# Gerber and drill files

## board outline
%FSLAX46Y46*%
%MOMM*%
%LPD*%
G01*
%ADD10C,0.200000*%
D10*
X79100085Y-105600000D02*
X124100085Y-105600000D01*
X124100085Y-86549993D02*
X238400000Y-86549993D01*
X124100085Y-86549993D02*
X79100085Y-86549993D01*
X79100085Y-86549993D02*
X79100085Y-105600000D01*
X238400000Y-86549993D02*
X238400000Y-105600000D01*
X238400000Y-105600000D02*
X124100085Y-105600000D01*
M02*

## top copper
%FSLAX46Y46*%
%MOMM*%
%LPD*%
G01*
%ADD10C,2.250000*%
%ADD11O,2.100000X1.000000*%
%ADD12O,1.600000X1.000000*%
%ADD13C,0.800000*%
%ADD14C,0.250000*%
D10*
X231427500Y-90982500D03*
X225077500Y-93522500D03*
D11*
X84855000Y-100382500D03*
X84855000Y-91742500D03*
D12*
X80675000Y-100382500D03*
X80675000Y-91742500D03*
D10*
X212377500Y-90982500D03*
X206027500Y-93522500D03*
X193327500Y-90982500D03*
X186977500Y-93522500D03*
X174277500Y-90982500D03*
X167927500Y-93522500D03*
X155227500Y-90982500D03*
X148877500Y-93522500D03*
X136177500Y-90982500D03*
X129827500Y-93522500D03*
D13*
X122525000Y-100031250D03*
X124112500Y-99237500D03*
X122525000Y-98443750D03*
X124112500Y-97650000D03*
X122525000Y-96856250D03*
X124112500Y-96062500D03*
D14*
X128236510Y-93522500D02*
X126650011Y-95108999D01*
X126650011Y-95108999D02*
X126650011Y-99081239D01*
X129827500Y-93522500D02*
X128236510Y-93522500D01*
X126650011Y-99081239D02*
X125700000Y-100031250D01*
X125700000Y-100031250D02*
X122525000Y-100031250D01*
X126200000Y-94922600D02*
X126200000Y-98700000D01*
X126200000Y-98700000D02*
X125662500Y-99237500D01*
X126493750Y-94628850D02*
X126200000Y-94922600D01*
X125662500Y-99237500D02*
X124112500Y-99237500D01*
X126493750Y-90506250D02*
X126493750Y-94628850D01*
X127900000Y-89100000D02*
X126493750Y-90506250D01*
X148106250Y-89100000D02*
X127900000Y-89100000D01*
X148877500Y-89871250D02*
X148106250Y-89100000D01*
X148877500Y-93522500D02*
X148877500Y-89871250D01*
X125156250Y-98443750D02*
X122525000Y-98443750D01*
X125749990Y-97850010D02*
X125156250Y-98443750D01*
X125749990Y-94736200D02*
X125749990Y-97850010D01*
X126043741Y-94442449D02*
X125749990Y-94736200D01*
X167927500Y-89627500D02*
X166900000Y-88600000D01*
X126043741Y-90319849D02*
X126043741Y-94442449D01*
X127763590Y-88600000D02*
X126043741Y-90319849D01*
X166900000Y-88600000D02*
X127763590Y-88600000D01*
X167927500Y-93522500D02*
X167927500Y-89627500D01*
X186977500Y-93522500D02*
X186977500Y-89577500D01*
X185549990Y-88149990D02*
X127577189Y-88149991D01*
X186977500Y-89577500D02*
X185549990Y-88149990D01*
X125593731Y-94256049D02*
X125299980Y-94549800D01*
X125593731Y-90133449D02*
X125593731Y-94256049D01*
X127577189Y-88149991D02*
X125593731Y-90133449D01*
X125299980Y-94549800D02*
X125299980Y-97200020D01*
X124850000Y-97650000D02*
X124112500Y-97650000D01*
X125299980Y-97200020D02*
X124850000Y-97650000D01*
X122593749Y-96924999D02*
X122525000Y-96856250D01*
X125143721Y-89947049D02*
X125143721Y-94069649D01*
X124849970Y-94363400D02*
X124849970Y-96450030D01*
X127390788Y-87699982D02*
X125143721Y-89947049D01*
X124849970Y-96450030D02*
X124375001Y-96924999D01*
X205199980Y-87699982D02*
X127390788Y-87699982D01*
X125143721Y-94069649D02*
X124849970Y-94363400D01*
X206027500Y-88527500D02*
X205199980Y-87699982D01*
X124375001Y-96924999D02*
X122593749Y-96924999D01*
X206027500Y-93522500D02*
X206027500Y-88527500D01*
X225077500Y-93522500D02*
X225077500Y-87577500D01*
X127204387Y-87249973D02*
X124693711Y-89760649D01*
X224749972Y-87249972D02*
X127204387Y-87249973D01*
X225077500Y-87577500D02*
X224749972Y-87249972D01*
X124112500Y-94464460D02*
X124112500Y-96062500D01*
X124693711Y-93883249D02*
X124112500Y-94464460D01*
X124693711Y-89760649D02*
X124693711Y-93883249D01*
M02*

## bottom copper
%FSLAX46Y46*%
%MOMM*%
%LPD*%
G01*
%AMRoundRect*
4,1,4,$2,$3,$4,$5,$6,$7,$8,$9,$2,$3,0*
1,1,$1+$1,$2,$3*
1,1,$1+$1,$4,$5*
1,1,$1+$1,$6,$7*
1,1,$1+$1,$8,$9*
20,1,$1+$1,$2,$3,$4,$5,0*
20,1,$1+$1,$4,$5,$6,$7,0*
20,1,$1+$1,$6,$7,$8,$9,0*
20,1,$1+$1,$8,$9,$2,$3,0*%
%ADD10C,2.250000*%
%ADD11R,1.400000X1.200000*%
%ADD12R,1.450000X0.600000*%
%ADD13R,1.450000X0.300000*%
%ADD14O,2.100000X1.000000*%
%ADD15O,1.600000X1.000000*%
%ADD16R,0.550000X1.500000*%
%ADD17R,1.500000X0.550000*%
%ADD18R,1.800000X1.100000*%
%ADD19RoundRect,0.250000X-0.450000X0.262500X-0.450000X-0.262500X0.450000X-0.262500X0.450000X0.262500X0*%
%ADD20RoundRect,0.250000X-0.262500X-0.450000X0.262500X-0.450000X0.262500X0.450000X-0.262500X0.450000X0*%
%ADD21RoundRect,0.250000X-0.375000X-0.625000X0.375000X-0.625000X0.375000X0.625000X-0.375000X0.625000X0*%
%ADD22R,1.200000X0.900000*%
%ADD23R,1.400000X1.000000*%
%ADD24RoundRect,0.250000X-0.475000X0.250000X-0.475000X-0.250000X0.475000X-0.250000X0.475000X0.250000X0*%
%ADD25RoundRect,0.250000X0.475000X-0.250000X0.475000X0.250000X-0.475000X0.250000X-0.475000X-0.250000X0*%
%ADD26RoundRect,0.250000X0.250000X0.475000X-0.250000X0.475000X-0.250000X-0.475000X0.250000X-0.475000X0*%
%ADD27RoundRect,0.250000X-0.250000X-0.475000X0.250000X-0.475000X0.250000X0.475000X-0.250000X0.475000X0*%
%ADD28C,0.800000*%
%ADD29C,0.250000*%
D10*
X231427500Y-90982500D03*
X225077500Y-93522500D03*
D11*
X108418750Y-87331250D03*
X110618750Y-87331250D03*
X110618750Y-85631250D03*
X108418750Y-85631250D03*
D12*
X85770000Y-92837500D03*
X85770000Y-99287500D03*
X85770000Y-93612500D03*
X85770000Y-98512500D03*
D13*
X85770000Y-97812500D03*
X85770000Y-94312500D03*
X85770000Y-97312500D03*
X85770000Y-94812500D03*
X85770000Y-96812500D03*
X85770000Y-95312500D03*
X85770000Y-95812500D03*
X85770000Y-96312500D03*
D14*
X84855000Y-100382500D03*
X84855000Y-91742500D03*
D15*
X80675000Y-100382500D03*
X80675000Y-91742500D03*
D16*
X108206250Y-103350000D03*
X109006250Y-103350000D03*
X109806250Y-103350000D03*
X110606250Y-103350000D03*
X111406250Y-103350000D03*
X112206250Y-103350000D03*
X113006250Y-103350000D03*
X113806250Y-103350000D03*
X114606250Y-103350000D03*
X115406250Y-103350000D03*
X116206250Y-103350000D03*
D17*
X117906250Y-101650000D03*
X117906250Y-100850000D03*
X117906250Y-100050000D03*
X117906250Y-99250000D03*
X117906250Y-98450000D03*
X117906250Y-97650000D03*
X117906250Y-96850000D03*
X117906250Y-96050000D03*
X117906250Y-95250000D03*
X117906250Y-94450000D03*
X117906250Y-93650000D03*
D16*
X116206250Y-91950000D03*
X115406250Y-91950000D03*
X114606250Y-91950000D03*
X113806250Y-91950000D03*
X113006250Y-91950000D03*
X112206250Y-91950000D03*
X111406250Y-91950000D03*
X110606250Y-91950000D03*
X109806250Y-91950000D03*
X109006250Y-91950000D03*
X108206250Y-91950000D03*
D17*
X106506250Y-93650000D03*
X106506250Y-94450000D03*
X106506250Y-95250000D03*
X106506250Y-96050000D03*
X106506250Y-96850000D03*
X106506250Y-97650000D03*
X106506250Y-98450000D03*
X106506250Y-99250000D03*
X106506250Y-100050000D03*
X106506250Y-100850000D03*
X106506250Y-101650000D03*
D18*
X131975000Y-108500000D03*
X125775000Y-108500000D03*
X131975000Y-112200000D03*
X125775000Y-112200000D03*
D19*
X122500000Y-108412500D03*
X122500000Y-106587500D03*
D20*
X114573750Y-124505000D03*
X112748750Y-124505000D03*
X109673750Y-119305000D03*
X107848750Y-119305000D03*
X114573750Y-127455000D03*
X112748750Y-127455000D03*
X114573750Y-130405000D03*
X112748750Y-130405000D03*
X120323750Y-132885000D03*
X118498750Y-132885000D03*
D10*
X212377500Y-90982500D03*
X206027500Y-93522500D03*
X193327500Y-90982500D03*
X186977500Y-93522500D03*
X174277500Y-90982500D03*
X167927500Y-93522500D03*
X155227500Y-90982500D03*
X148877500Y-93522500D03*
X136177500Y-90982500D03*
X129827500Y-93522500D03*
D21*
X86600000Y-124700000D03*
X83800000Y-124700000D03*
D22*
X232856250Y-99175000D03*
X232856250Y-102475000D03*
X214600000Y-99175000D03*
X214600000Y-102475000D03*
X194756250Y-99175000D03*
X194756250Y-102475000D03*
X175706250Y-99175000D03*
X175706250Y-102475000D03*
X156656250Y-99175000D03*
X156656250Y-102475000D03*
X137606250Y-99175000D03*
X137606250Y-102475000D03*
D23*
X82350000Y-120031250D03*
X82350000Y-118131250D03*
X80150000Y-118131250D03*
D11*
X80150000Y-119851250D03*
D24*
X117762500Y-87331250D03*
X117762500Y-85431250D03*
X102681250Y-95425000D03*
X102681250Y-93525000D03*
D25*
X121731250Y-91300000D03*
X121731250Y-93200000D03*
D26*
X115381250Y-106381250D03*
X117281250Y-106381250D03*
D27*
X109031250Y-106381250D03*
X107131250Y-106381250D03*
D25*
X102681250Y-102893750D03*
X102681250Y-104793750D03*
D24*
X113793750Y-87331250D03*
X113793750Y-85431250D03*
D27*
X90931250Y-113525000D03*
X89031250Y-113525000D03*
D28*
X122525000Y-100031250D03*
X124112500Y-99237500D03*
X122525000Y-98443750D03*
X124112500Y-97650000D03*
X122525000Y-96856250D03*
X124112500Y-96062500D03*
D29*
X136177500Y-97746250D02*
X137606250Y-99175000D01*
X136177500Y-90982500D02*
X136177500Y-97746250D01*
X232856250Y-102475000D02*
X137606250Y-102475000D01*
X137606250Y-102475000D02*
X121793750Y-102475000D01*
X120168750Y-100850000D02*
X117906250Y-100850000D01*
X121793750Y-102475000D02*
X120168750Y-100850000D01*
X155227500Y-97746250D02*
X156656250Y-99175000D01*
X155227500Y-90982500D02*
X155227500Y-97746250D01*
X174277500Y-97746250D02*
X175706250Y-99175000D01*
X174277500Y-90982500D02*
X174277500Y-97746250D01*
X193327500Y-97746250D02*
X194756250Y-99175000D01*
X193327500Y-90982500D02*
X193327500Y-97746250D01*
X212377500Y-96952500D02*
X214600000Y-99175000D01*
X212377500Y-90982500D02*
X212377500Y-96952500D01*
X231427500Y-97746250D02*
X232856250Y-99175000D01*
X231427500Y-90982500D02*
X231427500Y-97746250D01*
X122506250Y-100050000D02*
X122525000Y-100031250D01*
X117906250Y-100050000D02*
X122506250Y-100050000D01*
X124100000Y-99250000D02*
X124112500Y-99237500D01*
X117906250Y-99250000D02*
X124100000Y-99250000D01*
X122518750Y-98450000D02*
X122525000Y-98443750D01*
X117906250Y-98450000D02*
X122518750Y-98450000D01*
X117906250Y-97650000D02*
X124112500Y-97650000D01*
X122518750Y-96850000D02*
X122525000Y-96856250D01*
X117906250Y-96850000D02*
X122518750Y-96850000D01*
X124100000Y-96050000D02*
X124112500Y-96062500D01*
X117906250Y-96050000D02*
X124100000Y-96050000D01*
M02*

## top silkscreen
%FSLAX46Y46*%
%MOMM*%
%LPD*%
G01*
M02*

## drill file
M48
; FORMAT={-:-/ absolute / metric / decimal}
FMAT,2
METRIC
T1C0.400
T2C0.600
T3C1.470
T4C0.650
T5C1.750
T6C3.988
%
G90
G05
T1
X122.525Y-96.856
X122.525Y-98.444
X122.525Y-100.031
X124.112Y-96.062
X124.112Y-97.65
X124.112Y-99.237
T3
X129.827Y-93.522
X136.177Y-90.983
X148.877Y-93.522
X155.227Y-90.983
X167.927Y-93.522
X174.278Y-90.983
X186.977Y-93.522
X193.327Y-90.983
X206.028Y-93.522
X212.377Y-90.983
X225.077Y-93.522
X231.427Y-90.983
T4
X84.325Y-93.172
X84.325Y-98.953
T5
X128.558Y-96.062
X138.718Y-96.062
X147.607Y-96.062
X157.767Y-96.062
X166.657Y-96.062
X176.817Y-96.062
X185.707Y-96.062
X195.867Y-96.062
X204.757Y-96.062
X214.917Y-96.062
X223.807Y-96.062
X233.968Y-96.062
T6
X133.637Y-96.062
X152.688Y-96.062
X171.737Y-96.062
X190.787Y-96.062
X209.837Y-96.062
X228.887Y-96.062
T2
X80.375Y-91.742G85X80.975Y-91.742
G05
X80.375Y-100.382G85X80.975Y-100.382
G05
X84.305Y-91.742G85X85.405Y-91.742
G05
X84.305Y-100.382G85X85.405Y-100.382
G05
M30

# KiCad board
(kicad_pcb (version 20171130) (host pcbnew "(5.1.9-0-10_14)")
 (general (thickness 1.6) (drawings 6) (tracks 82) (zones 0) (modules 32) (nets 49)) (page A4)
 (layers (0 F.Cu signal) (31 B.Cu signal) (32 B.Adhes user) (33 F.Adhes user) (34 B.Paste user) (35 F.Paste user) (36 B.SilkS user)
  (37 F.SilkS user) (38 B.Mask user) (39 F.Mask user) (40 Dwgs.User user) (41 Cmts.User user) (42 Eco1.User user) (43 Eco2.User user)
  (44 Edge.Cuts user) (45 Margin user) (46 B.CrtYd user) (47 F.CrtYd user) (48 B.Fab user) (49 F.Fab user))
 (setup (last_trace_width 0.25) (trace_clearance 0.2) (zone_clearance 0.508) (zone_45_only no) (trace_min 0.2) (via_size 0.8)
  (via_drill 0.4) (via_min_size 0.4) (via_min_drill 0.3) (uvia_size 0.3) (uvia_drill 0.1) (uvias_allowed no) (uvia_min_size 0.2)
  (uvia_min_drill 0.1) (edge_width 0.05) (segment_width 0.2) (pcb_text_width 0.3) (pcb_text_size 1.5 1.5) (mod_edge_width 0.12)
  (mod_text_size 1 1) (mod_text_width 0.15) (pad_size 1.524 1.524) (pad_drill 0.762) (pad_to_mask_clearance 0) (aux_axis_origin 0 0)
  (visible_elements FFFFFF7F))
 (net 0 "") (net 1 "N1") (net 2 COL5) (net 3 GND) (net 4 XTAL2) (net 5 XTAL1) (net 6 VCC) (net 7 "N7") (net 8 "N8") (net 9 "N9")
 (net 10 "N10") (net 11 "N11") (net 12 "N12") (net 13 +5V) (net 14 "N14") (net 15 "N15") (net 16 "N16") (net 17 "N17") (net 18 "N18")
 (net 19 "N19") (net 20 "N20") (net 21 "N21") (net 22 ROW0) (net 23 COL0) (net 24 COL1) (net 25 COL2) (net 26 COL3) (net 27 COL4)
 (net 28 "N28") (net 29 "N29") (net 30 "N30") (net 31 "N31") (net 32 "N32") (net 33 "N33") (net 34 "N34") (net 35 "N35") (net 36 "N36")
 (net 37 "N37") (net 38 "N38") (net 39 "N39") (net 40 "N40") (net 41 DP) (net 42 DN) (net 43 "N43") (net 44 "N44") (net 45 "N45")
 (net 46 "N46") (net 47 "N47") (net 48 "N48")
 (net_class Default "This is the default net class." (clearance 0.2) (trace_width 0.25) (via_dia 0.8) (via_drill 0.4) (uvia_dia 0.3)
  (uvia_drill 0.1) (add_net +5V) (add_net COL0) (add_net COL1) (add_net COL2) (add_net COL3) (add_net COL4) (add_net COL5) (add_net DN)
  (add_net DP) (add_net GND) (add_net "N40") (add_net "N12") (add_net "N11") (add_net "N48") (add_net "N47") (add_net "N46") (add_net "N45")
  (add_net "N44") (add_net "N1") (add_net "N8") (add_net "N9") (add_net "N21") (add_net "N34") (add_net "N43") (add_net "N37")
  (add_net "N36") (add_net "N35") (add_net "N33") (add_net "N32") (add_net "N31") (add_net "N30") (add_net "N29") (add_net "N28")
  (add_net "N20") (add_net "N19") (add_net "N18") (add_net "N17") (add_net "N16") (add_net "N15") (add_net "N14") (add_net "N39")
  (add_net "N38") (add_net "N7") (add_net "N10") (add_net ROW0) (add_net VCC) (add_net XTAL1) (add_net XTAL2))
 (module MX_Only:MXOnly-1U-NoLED (layer F.Cu) (at 228.8875 96.0625)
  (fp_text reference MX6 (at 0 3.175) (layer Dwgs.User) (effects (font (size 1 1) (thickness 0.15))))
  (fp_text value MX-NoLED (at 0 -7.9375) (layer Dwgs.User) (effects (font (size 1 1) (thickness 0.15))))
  (pad 2 thru_hole circle (at 2.54 -5.08) (size 2.25 2.25) (drill 1.47) (layers *.Cu B.Mask) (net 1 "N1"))
  (pad "" np_thru_hole circle (at 0 0) (size 3.9878 3.9878) (drill 3.9878) (layers *.Cu *.Mask))
  (pad 1 thru_hole circle (at -3.81 -2.54) (size 2.25 2.25) (drill 1.47) (layers *.Cu B.Mask) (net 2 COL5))
  (pad "" np_thru_hole circle (at -5.08 0 48.0996) (size 1.75 1.75) (drill 1.75) (layers *.Cu *.Mask))
  (pad "" np_thru_hole circle (at 5.08 0 48.0996) (size 1.75 1.75) (drill 1.75) (layers *.Cu *.Mask)))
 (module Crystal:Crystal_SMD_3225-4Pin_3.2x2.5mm (layer B.Cu) (at 109.51875 86.48125)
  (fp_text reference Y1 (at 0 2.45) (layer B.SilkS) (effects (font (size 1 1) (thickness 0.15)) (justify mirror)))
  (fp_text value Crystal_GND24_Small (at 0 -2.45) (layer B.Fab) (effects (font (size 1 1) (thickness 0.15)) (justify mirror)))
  (pad 4 smd rect (at -1.1 0.85) (size 1.4 1.2) (layers B.Cu B.Paste B.Mask) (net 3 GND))
  (pad 3 smd rect (at 1.1 0.85) (size 1.4 1.2) (layers B.Cu B.Paste B.Mask) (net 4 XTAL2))
  (pad 2 smd rect (at 1.1 -0.85) (size 1.4 1.2) (layers B.Cu B.Paste B.Mask) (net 3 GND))
  (pad 1 smd rect (at -1.1 -0.85) (size 1.4 1.2) (layers B.Cu B.Paste B.Mask) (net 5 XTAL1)))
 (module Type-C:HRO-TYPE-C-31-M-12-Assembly (layer B.Cu) (at 78.075 96.0625 90)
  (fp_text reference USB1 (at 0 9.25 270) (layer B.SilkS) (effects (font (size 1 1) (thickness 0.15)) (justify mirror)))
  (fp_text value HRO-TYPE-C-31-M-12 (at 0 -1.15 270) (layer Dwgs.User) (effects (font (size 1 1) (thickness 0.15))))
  (pad 12 smd rect (at 3.225 7.695 90) (size 0.6 1.45) (layers B.Cu B.Paste B.Mask) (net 3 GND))
  (pad 1 smd rect (at -3.225 7.695 90) (size 0.6 1.45) (layers B.Cu B.Paste B.Mask) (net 3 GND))
  (pad 11 smd rect (at 2.45 7.695 90) (size 0.6 1.45) (layers B.Cu B.Paste B.Mask) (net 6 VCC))
  (pad 2 smd rect (at -2.45 7.695 90) (size 0.6 1.45) (layers B.Cu B.Paste B.Mask) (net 6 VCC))
  (pad 3 smd rect (at -1.75 7.695 90) (size 0.3 1.45) (layers B.Cu B.Paste B.Mask) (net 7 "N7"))
  (pad 10 smd rect (at 1.75 7.695 90) (size 0.3 1.45) (layers B.Cu B.Paste B.Mask) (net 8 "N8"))
  (pad 4 smd rect (at -1.25 7.695 90) (size 0.3 1.45) (layers B.Cu B.Paste B.Mask) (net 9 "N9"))
  (pad 9 smd rect (at 1.25 7.695 90) (size 0.3 1.45) (layers B.Cu B.Paste B.Mask) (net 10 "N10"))
  (pad 5 smd rect (at -0.75 7.695 90) (size 0.3 1.45) (layers B.Cu B.Paste B.Mask) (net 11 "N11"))
  (pad 8 smd rect (at 0.75 7.695 90) (size 0.3 1.45) (layers B.Cu B.Paste B.Mask) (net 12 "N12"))
  (pad 7 smd rect (at 0.25 7.695 90) (size 0.3 1.45) (layers B.Cu B.Paste B.Mask) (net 11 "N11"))
  (pad 6 smd rect (at -0.25 7.695 90) (size 0.3 1.45) (layers B.Cu B.Paste B.Mask) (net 12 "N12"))
  (pad "" np_thru_hole circle (at 2.89 6.25 90) (size 0.65 0.65) (drill 0.65) (layers *.Cu *.Mask))
  (pad "" np_thru_hole circle (at -2.89 6.25 90) (size 0.65 0.65) (drill 0.65) (layers *.Cu *.Mask))
  (pad 13 thru_hole oval (at -4.32 6.78 90) (size 1 2.1) (drill oval 0.6 1.7) (layers *.Cu *.Mask) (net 3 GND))
  (pad 13 thru_hole oval (at 4.32 6.78 90) (size 1 2.1) (drill oval 0.6 1.7) (layers *.Cu *.Mask) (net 3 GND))
  (pad 13 thru_hole oval (at -4.32 2.6 90) (size 1 1.6) (drill oval 0.6 1.2) (layers *.Cu *.Mask) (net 3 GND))
  (pad 13 thru_hole oval (at 4.32 2.6 90) (size 1 1.6) (drill oval 0.6 1.2) (layers *.Cu *.Mask) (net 3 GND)))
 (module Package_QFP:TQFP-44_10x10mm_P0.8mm (layer B.Cu) (at 112.20625 97.65)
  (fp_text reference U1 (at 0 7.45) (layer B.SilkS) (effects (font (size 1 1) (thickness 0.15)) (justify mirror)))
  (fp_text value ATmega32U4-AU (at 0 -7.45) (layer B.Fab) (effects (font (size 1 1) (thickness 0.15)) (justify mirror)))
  (pad 44 smd rect (at -4 5.7 270) (size 1.5 0.55) (layers B.Cu B.Paste B.Mask) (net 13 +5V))
  (pad 43 smd rect (at -3.2 5.7 270) (size 1.5 0.55) (layers B.Cu B.Paste B.Mask) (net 3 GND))
  (pad 42 smd rect (at -2.4 5.7 270) (size 1.5 0.55) (layers B.Cu B.Paste B.Mask) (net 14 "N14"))
  (pad 41 smd rect (at -1.6 5.7 270) (size 1.5 0.55) (layers B.Cu B.Paste B.Mask) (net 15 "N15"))
  (pad 40 smd rect (at -0.8 5.7 270) (size 1.5 0.55) (layers B.Cu B.Paste B.Mask) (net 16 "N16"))
  (pad 39 smd rect (at 0 5.7 270) (size 1.5 0.55) (layers B.Cu B.Paste B.Mask) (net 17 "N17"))
  (pad 38 smd rect (at 0.8 5.7 270) (size 1.5 0.55) (layers B.Cu B.Paste B.Mask) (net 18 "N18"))
  (pad 37 smd rect (at 1.6 5.7 270) (size 1.5 0.55) (layers B.Cu B.Paste B.Mask) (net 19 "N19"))
  (pad 36 smd rect (at 2.4 5.7 270) (size 1.5 0.55) (layers B.Cu B.Paste B.Mask) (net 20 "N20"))
  (pad 35 smd rect (at 3.2 5.7 270) (size 1.5 0.55) (layers B.Cu B.Paste B.Mask) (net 3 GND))
  (pad 34 smd rect (at 4 5.7 270) (size 1.5 0.55) (layers B.Cu B.Paste B.Mask) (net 13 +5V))
  (pad 33 smd rect (at 5.7 4) (size 1.5 0.55) (layers B.Cu B.Paste B.Mask) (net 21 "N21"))
  (pad 32 smd rect (at 5.7 3.2) (size 1.5 0.55) (layers B.Cu B.Paste B.Mask) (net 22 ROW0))
  (pad 31 smd rect (at 5.7 2.4) (size 1.5 0.55) (layers B.Cu B.Paste B.Mask) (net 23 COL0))
  (pad 30 smd rect (at 5.7 1.6) (size 1.5 0.55) (layers B.Cu B.Paste B.Mask) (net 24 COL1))
  (pad 29 smd rect (at 5.7 0.8) (size 1.5 0.55) (layers B.Cu B.Paste B.Mask) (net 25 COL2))
  (pad 28 smd rect (at 5.7 0) (size 1.5 0.55) (layers B.Cu B.Paste B.Mask) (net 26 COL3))
  (pad 27 smd rect (at 5.7 -0.8) (size 1.5 0.55) (layers B.Cu B.Paste B.Mask) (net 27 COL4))
  (pad 26 smd rect (at 5.7 -1.6) (size 1.5 0.55) (layers B.Cu B.Paste B.Mask) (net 2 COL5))
  (pad 25 smd rect (at 5.7 -2.4) (size 1.5 0.55) (layers B.Cu B.Paste B.Mask) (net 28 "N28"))
  (pad 24 smd rect (at 5.7 -3.2) (size 1.5 0.55) (layers B.Cu B.Paste B.Mask) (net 13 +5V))
  (pad 23 smd rect (at 5.7 -4) (size 1.5 0.55) (layers B.Cu B.Paste B.Mask) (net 3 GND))
  (pad 22 smd rect (at 4 -5.7 270) (size 1.5 0.55) (layers B.Cu B.Paste B.Mask) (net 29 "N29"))
  (pad 21 smd rect (at 3.2 -5.7 270) (size 1.5 0.55) (layers B.Cu B.Paste B.Mask) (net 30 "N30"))
  (pad 20 smd rect (at 2.4 -5.7 270) (size 1.5 0.55) (layers B.Cu B.Paste B.Mask) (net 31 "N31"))
  (pad 19 smd rect (at 1.6 -5.7 270) (size 1.5 0.55) (layers B.Cu B.Paste B.Mask) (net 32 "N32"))
  (pad 18 smd rect (at 0.8 -5.7 270) (size 1.5 0.55) (layers B.Cu B.Paste B.Mask) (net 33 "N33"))
  (pad 17 smd rect (at 0 -5.7 270) (size 1.5 0.55) (layers B.Cu B.Paste B.Mask) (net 5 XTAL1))
  (pad 16 smd rect (at -0.8 -5.7 270) (size 1.5 0.55) (layers B.Cu B.Paste B.Mask) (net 4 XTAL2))
  (pad 15 smd rect (at -1.6 -5.7 270) (size 1.5 0.55) (layers B.Cu B.Paste B.Mask) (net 3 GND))
  (pad 14 smd rect (at -2.4 -5.7 270) (size 1.5 0.55) (layers B.Cu B.Paste B.Mask) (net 13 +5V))
  (pad 13 smd rect (at -3.2 -5.7 270) (size 1.5 0.55) (layers B.Cu B.Paste B.Mask) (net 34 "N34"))
  (pad 12 smd rect (at -4 -5.7 270) (size 1.5 0.55) (layers B.Cu B.Paste B.Mask) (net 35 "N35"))
  (pad 11 smd rect (at -5.7 -4) (size 1.5 0.55) (layers B.Cu B.Paste B.Mask) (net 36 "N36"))
  (pad 10 smd rect (at -5.7 -3.2) (size 1.5 0.55) (layers B.Cu B.Paste B.Mask) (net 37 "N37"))
  (pad 9 smd rect (at -5.7 -2.4) (size 1.5 0.55) (layers B.Cu B.Paste B.Mask) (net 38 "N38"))
  (pad 8 smd rect (at -5.7 -1.6) (size 1.5 0.55) (layers B.Cu B.Paste B.Mask) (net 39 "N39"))
  (pad 7 smd rect (at -5.7 -0.8) (size 1.5 0.55) (layers B.Cu B.Paste B.Mask) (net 13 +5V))
  (pad 6 smd rect (at -5.7 0) (size 1.5 0.55) (layers B.Cu B.Paste B.Mask) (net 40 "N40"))
  (pad 5 smd rect (at -5.7 0.8) (size 1.5 0.55) (layers B.Cu B.Paste B.Mask) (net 3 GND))
  (pad 4 smd rect (at -5.7 1.6) (size 1.5 0.55) (layers B.Cu B.Paste B.Mask) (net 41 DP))
  (pad 3 smd rect (at -5.7 2.4) (size 1.5 0.55) (layers B.Cu B.Paste B.Mask) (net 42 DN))
  (pad 2 smd rect (at -5.7 3.2) (size 1.5 0.55) (layers B.Cu B.Paste B.Mask) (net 13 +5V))
  (pad 1 smd rect (at -5.7 4) (size 1.5 0.55) (layers B.Cu B.Paste B.Mask) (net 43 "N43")))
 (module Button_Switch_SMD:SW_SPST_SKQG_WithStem (layer B.Cu) (at 128.875 110.35)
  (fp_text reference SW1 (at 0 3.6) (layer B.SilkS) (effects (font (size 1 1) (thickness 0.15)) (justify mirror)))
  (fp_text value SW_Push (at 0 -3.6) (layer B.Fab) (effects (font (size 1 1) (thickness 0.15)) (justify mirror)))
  (pad 2 smd rect (at 3.1 -1.85) (size 1.8 1.1) (layers B.Cu B.Paste B.Mask) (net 34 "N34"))
  (pad 2 smd rect (at -3.1 -1.85) (size 1.8 1.1) (layers B.Cu B.Paste B.Mask) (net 34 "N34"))
  (pad 1 smd rect (at 3.1 1.85) (size 1.8 1.1) (layers B.Cu B.Paste B.Mask) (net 3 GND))
  (pad 1 smd rect (at -3.1 1.85) (size 1.8 1.1) (layers B.Cu B.Paste B.Mask) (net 3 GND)))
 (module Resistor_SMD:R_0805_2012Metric (layer B.Cu) (at 122.5 107.5 270)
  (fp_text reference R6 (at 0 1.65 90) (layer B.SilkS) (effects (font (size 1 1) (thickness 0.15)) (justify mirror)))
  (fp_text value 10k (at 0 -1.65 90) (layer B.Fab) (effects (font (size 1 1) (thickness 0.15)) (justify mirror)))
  (pad 2 smd roundrect (at 0.9125 0 270) (size 1.025 1.4) (layers B.Cu B.Paste B.Mask) (roundrect_rratio 0.243902) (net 34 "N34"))
  (pad 1 smd roundrect (at -0.9125 0 270) (size 1.025 1.4) (layers B.Cu B.Paste B.Mask) (roundrect_rratio 0.243902) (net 13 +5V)))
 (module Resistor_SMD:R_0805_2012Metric (layer B.Cu) (at 113.66125 124.505)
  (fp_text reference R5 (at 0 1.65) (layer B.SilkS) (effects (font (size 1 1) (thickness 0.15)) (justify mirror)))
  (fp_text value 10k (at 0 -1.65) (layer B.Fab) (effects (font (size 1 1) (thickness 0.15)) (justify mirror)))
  (pad 2 smd roundrect (at 0.9125 0) (size 1.025 1.4) (layers B.Cu B.Paste B.Mask) (roundrect_rratio 0.243902) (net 21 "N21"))
  (pad 1 smd roundrect (at -0.9125 0) (size 1.025 1.4) (layers B.Cu B.Paste B.Mask) (roundrect_rratio 0.243902) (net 3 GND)))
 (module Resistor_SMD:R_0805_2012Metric (layer B.Cu) (at 108.76125 119.305)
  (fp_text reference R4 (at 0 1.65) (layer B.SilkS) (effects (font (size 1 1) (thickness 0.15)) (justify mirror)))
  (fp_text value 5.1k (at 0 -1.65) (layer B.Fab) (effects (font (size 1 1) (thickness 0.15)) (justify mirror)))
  (pad 2 smd roundrect (at 0.9125 0) (size 1.025 1.4) (layers B.Cu B.Paste B.Mask) (roundrect_rratio 0.243902) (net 9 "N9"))
  (pad 1 smd roundrect (at -0.9125 0) (size 1.025 1.4) (layers B.Cu B.Paste B.Mask) (roundrect_rratio 0.243902) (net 3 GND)))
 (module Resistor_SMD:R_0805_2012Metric (layer B.Cu) (at 113.66125 127.455)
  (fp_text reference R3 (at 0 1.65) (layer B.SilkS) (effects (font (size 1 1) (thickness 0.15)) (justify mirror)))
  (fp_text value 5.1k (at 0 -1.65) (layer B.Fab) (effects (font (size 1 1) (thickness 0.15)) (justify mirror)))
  (pad 2 smd roundrect (at 0.9125 0) (size 1.025 1.4) (layers B.Cu B.Paste B.Mask) (roundrect_rratio 0.243902) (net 8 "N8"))
  (pad 1 smd roundrect (at -0.9125 0) (size 1.025 1.4) (layers B.Cu B.Paste B.Mask) (roundrect_rratio 0.243902) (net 3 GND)))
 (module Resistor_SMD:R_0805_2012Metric (layer B.Cu) (at 113.66125 130.405)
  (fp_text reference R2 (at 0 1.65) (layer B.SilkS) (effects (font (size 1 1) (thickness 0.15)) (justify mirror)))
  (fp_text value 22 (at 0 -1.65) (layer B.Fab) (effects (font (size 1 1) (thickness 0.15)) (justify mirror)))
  (pad 2 smd roundrect (at 0.9125 0) (size 1.025 1.4) (layers B.Cu B.Paste B.Mask) (roundrect_rratio 0.243902) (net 41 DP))
  (pad 1 smd roundrect (at -0.9125 0) (size 1.025 1.4) (layers B.Cu B.Paste B.Mask) (roundrect_rratio 0.243902) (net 12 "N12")))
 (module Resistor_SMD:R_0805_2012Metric (layer B.Cu) (at 119.41125 132.885)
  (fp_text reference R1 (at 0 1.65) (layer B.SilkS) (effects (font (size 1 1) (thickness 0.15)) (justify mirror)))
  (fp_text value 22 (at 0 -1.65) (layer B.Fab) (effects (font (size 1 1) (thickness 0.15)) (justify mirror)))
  (pad 2 smd roundrect (at 0.9125 0) (size 1.025 1.4) (layers B.Cu B.Paste B.Mask) (roundrect_rratio 0.243902) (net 42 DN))
  (pad 1 smd roundrect (at -0.9125 0) (size 1.025 1.4) (layers B.Cu B.Paste B.Mask) (roundrect_rratio 0.243902) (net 11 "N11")))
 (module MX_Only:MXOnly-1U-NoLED (layer F.Cu) (at 209.8375 96.0625)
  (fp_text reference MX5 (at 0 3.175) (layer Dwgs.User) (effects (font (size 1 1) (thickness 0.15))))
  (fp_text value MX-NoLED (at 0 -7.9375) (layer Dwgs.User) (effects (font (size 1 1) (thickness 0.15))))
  (pad 2 thru_hole circle (at 2.54 -5.08) (size 2.25 2.25) (drill 1.47) (layers *.Cu B.Mask) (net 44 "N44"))
  (pad "" np_thru_hole circle (at 0 0) (size 3.9878 3.9878) (drill 3.9878) (layers *.Cu *.Mask))
  (pad 1 thru_hole circle (at -3.81 -2.54) (size 2.25 2.25) (drill 1.47) (layers *.Cu B.Mask) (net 27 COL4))
  (pad "" np_thru_hole circle (at -5.08 0 48.0996) (size 1.75 1.75) (drill 1.75) (layers *.Cu *.Mask))
  (pad "" np_thru_hole circle (at 5.08 0 48.0996) (size 1.75 1.75) (drill 1.75) (layers *.Cu *.Mask)))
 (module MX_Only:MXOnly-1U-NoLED (layer F.Cu) (at 190.7875 96.0625)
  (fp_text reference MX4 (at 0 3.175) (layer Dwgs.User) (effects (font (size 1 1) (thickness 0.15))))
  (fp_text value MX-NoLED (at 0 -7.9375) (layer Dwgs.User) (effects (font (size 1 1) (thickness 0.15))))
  (pad 2 thru_hole circle (at 2.54 -5.08) (size 2.25 2.25) (drill 1.47) (layers *.Cu B.Mask) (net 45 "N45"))
  (pad "" np_thru_hole circle (at 0 0) (size 3.9878 3.9878) (drill 3.9878) (layers *.Cu *.Mask))
  (pad 1 thru_hole circle (at -3.81 -2.54) (size 2.25 2.25) (drill 1.47) (layers *.Cu B.Mask) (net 26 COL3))
  (pad "" np_thru_hole circle (at -5.08 0 48.0996) (size 1.75 1.75) (drill 1.75) (layers *.Cu *.Mask))
  (pad "" np_thru_hole circle (at 5.08 0 48.0996) (size 1.75 1.75) (drill 1.75) (layers *.Cu *.Mask)))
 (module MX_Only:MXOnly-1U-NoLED (layer F.Cu) (at 171.7375 96.0625)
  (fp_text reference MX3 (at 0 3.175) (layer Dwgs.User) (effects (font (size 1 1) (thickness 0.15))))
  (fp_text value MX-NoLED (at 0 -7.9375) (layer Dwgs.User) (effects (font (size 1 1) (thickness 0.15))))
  (pad 2 thru_hole circle (at 2.54 -5.08) (size 2.25 2.25) (drill 1.47) (layers *.Cu B.Mask) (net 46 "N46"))
  (pad "" np_thru_hole circle (at 0 0) (size 3.9878 3.9878) (drill 3.9878) (layers *.Cu *.Mask))
  (pad 1 thru_hole circle (at -3.81 -2.54) (size 2.25 2.25) (drill 1.47) (layers *.Cu B.Mask) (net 25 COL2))
  (pad "" np_thru_hole circle (at -5.08 0 48.0996) (size 1.75 1.75) (drill 1.75) (layers *.Cu *.Mask))
  (pad "" np_thru_hole circle (at 5.08 0 48.0996) (size 1.75 1.75) (drill 1.75) (layers *.Cu *.Mask)))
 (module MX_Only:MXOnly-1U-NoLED (layer F.Cu) (at 152.6875 96.0625)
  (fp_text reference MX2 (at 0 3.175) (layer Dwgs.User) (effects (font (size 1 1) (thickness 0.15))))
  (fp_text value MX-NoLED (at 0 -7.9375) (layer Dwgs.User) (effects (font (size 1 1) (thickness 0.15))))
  (pad 2 thru_hole circle (at 2.54 -5.08) (size 2.25 2.25) (drill 1.47) (layers *.Cu B.Mask) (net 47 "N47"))
  (pad "" np_thru_hole circle (at 0 0) (size 3.9878 3.9878) (drill 3.9878) (layers *.Cu *.Mask))
  (pad 1 thru_hole circle (at -3.81 -2.54) (size 2.25 2.25) (drill 1.47) (layers *.Cu B.Mask) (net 24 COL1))
  (pad "" np_thru_hole circle (at -5.08 0 48.0996) (size 1.75 1.75) (drill 1.75) (layers *.Cu *.Mask))
  (pad "" np_thru_hole circle (at 5.08 0 48.0996) (size 1.75 1.75) (drill 1.75) (layers *.Cu *.Mask)))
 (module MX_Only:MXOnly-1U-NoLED (layer F.Cu) (at 133.6375 96.0625)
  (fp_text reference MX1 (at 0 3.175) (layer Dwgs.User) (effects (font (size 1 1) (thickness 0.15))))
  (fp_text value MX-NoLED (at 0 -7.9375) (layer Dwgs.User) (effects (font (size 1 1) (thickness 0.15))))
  (pad 2 thru_hole circle (at 2.54 -5.08) (size 2.25 2.25) (drill 1.47) (layers *.Cu B.Mask) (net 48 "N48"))
  (pad "" np_thru_hole circle (at 0 0) (size 3.9878 3.9878) (drill 3.9878) (layers *.Cu *.Mask))
  (pad 1 thru_hole circle (at -3.81 -2.54) (size 2.25 2.25) (drill 1.47) (layers *.Cu B.Mask) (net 23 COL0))
  (pad "" np_thru_hole circle (at -5.08 0 48.0996) (size 1.75 1.75) (drill 1.75) (layers *.Cu *.Mask))
  (pad "" np_thru_hole circle (at 5.08 0 48.0996) (size 1.75 1.75) (drill 1.75) (layers *.Cu *.Mask)))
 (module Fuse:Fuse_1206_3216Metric (layer B.Cu) (at 85.2 124.7)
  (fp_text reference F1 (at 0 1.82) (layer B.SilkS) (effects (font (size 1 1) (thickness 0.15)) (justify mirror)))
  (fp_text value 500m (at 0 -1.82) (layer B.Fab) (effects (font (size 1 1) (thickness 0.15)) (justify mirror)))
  (pad 2 smd roundrect (at 1.4 0) (size 1.25 1.75) (layers B.Cu B.Paste B.Mask) (roundrect_rratio 0.2) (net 6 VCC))
  (pad 1 smd roundrect (at -1.4 0) (size 1.25 1.75) (layers B.Cu B.Paste B.Mask) (roundrect_rratio 0.2) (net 13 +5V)))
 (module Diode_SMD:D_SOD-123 (layer B.Cu) (at 232.85625 100.825 90)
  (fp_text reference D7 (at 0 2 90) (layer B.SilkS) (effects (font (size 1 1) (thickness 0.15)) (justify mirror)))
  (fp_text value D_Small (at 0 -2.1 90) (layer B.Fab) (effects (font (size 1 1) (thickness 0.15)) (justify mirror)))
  (pad 2 smd rect (at 1.65 0 90) (size 0.9 1.2) (layers B.Cu B.Paste B.Mask) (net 1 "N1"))
  (pad 1 smd rect (at -1.65 0 90) (size 0.9 1.2) (layers B.Cu B.Paste B.Mask) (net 22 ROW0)))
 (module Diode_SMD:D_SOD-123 (layer B.Cu) (at 214.6 100.825 90)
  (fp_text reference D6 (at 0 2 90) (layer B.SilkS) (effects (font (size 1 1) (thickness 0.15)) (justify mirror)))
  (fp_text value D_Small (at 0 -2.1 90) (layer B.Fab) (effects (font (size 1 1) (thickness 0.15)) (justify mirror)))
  (pad 2 smd rect (at 1.65 0 90) (size 0.9 1.2) (layers B.Cu B.Paste B.Mask) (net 44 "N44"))
  (pad 1 smd rect (at -1.65 0 90) (size 0.9 1.2) (layers B.Cu B.Paste B.Mask) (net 22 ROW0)))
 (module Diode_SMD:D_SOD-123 (layer B.Cu) (at 194.75625 100.825 90)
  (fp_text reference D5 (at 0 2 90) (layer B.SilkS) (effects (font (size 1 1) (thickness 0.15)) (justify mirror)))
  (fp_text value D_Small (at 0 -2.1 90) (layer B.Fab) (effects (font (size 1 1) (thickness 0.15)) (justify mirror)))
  (pad 2 smd rect (at 1.65 0 90) (size 0.9 1.2) (layers B.Cu B.Paste B.Mask) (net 45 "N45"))
  (pad 1 smd rect (at -1.65 0 90) (size 0.9 1.2) (layers B.Cu B.Paste B.Mask) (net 22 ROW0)))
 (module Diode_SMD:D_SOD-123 (layer B.Cu) (at 175.70625 100.825 90)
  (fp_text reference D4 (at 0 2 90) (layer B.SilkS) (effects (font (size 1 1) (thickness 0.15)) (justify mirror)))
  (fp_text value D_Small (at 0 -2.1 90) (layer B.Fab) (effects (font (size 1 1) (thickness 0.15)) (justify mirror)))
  (pad 2 smd rect (at 1.65 0 90) (size 0.9 1.2) (layers B.Cu B.Paste B.Mask) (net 46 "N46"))
  (pad 1 smd rect (at -1.65 0 90) (size 0.9 1.2) (layers B.Cu B.Paste B.Mask) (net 22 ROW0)))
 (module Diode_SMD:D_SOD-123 (layer B.Cu) (at 156.65625 100.825 90)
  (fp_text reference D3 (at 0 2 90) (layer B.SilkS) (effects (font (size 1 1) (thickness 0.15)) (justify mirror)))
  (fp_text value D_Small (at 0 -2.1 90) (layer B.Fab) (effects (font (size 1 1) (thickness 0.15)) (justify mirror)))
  (pad 2 smd rect (at 1.65 0 90) (size 0.9 1.2) (layers B.Cu B.Paste B.Mask) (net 47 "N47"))
  (pad 1 smd rect (at -1.65 0 90) (size 0.9 1.2) (layers B.Cu B.Paste B.Mask) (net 22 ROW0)))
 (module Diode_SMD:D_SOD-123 (layer B.Cu) (at 137.60625 100.825 90)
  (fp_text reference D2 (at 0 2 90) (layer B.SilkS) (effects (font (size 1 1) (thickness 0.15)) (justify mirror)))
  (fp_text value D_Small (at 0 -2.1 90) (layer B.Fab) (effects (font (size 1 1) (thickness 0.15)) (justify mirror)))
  (pad 2 smd rect (at 1.65 0 90) (size 0.9 1.2) (layers B.Cu B.Paste B.Mask) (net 48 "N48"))
  (pad 1 smd rect (at -1.65 0 90) (size 0.9 1.2) (layers B.Cu B.Paste B.Mask) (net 22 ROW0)))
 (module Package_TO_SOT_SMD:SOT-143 (layer B.Cu) (at 81.25 119.08125)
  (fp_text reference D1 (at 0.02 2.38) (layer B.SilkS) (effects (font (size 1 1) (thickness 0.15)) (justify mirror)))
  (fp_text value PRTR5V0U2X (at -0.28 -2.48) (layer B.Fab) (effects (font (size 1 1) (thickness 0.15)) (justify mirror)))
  (pad 4 smd rect (at 1.1 0.95 90) (size 1 1.4) (layers B.Cu B.Paste B.Mask) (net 6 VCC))
  (pad 3 smd rect (at 1.1 -0.95 90) (size 1 1.4) (layers B.Cu B.Paste B.Mask) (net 11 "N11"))
  (pad 2 smd rect (at -1.1 -0.95 90) (size 1 1.4) (layers B.Cu B.Paste B.Mask) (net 12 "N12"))
  (pad 1 smd rect (at -1.1 0.77 90) (size 1.2 1.4) (layers B.Cu B.Paste B.Mask) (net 3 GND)))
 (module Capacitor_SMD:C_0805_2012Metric (layer B.Cu) (at 117.7625 86.38125 270)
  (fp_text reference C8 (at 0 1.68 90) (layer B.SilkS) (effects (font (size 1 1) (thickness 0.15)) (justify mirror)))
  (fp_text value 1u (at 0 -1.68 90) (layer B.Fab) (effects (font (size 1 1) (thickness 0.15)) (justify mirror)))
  (pad 2 smd roundrect (at 0.95 0 270) (size 1 1.45) (layers B.Cu B.Paste B.Mask) (roundrect_rratio 0.25) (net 3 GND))
  (pad 1 smd roundrect (at -0.95 0 270) (size 1 1.45) (layers B.Cu B.Paste B.Mask) (roundrect_rratio 0.25) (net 40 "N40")))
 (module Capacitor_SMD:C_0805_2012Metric (layer B.Cu) (at 102.68125 94.475 270)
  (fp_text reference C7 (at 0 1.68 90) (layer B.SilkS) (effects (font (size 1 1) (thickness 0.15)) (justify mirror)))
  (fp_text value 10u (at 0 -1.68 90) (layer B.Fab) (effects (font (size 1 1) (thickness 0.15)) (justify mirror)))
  (pad 2 smd roundrect (at 0.95 0 270) (size 1 1.45) (layers B.Cu B.Paste B.Mask) (roundrect_rratio 0.25) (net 3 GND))
  (pad 1 smd roundrect (at -0.95 0 270) (size 1 1.45) (layers B.Cu B.Paste B.Mask) (roundrect_rratio 0.25) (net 13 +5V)))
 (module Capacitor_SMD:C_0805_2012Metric (layer B.Cu) (at 121.73125 92.25 90)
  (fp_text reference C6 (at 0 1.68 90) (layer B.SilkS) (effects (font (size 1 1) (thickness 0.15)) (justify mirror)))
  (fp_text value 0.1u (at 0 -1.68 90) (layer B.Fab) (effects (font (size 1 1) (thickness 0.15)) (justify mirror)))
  (pad 2 smd roundrect (at 0.95 0 90) (size 1 1.45) (layers B.Cu B.Paste B.Mask) (roundrect_rratio 0.25) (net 3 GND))
  (pad 1 smd roundrect (at -0.95 0 90) (size 1 1.45) (layers B.Cu B.Paste B.Mask) (roundrect_rratio 0.25) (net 13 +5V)))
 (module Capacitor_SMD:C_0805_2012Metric (layer B.Cu) (at 116.33125 106.38125 180)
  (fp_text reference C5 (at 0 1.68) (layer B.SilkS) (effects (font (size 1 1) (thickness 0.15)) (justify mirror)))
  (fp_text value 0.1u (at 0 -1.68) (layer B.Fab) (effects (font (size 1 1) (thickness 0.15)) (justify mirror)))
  (pad 2 smd roundrect (at 0.95 0 180) (size 1 1.45) (layers B.Cu B.Paste B.Mask) (roundrect_rratio 0.25) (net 3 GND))
  (pad 1 smd roundrect (at -0.95 0 180) (size 1 1.45) (layers B.Cu B.Paste B.Mask) (roundrect_rratio 0.25) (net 13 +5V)))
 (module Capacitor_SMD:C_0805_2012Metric (layer B.Cu) (at 108.08125 106.38125)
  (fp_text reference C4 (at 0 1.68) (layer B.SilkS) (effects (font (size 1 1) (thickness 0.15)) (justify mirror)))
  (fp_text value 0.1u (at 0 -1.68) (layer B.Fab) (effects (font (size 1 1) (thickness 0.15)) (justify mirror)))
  (pad 2 smd roundrect (at 0.95 0) (size 1 1.45) (layers B.Cu B.Paste B.Mask) (roundrect_rratio 0.25) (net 3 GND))
  (pad 1 smd roundrect (at -0.95 0) (size 1 1.45) (layers B.Cu B.Paste B.Mask) (roundrect_rratio 0.25) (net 13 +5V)))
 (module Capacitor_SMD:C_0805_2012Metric (layer B.Cu) (at 102.68125 103.84375 90)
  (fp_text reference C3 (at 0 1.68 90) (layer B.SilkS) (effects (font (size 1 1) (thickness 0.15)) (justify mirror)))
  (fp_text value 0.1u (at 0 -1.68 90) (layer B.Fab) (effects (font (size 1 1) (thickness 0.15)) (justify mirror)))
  (pad 2 smd roundrect (at 0.95 0 90) (size 1 1.45) (layers B.Cu B.Paste B.Mask) (roundrect_rratio 0.25) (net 3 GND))
  (pad 1 smd roundrect (at -0.95 0 90) (size 1 1.45) (layers B.Cu B.Paste B.Mask) (roundrect_rratio 0.25) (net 13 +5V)))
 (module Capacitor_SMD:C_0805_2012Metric (layer B.Cu) (at 113.79375 86.38125 270)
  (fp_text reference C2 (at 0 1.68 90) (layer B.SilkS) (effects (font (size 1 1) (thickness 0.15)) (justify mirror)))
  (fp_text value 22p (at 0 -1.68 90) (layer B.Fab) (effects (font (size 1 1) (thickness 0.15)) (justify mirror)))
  (pad 2 smd roundrect (at 0.95 0 270) (size 1 1.45) (layers B.Cu B.Paste B.Mask) (roundrect_rratio 0.25) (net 3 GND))
  (pad 1 smd roundrect (at -0.95 0 270) (size 1 1.45) (layers B.Cu B.Paste B.Mask) (roundrect_rratio 0.25) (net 4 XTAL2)))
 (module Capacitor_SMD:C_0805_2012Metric (layer B.Cu) (at 89.98125 113.525)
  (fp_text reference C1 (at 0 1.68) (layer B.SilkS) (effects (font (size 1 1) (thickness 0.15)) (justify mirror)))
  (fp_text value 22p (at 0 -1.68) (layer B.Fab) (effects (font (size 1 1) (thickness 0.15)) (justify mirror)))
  (pad 2 smd roundrect (at 0.95 0) (size 1 1.45) (layers B.Cu B.Paste B.Mask) (roundrect_rratio 0.25) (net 3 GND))
  (pad 1 smd roundrect (at -0.95 0) (size 1 1.45) (layers B.Cu B.Paste B.Mask) (roundrect_rratio 0.25) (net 5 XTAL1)))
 (gr_line (start 79.100085 105.6) (end 124.100085 105.6) (layer Edge.Cuts) (width 0.2))
 (gr_line (start 124.100085 86.549993) (end 238.4 86.549993) (layer Edge.Cuts) (width 0.2))
 (gr_line (start 124.100085 86.549993) (end 79.100085 86.549993) (layer Edge.Cuts) (width 0.2))
 (gr_line (start 79.100085 86.549993) (end 79.100085 105.6) (layer Edge.Cuts) (width 0.2))
 (gr_line (start 238.4 86.549993) (end 238.4 105.6) (layer Edge.Cuts) (width 0.2))
 (gr_line (start 238.4 105.6) (end 124.100085 105.6) (layer Edge.Cuts) (width 0.2))
 (segment (start 136.1775 97.74625) (end 137.60625 99.175) (width 0.25) (layer B.Cu) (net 48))
 (segment (start 136.1775 90.9825) (end 136.1775 97.74625) (width 0.25) (layer B.Cu) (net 48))
 (segment (start 232.85625 102.475) (end 137.60625 102.475) (width 0.25) (layer B.Cu) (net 22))
 (segment (start 137.60625 102.475) (end 121.79375 102.475) (width 0.25) (layer B.Cu) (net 22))
 (segment (start 120.16875 100.85) (end 117.90625 100.85) (width 0.25) (layer B.Cu) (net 22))
 (segment (start 121.79375 102.475) (end 120.16875 100.85) (width 0.25) (layer B.Cu) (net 22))
 (segment (start 155.2275 97.74625) (end 156.65625 99.175) (width 0.25) (layer B.Cu) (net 47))
 (segment (start 155.2275 90.9825) (end 155.2275 97.74625) (width 0.25) (layer B.Cu) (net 47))
 (segment (start 174.2775 97.74625) (end 175.70625 99.175) (width 0.25) (layer B.Cu) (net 46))
 (segment (start 174.2775 90.9825) (end 174.2775 97.74625) (width 0.25) (layer B.Cu) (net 46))
 (segment (start 193.3275 97.74625) (end 194.75625 99.175) (width 0.25) (layer B.Cu) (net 45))
 (segment (start 193.3275 90.9825) (end 193.3275 97.74625) (width 0.25) (layer B.Cu) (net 45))
 (segment (start 212.3775 96.9525) (end 214.6 99.175) (width 0.25) (layer B.Cu) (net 44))
 (segment (start 212.3775 90.9825) (end 212.3775 96.9525) (width 0.25) (layer B.Cu) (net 44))
 (segment (start 231.4275 97.74625) (end 232.85625 99.175) (width 0.25) (layer B.Cu) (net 1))
 (segment (start 231.4275 90.9825) (end 231.4275 97.74625) (width 0.25) (layer B.Cu) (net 1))
 (via (at 122.525 100.03125) (size 0.8) (drill 0.4) (layers F.Cu B.Cu) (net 23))
 (segment (start 122.50625 100.05) (end 122.525 100.03125) (width 0.25) (layer B.Cu) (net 23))
 (segment (start 117.90625 100.05) (end 122.50625 100.05) (width 0.25) (layer B.Cu) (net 23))
 (segment (start 128.23651 93.5225) (end 126.650011 95.108999) (width 0.25) (layer F.Cu) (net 23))
 (segment (start 126.650011 95.108999) (end 126.650011 99.081239) (width 0.25) (layer F.Cu) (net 23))
 (segment (start 129.8275 93.5225) (end 128.23651 93.5225) (width 0.25) (layer F.Cu) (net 23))
 (segment (start 126.650011 99.081239) (end 125.7 100.03125) (width 0.25) (layer F.Cu) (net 23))
 (segment (start 125.7 100.03125) (end 122.525 100.03125) (width 0.25) (layer F.Cu) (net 23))
 (segment (start 124.1 99.25) (end 124.1125 99.2375) (width 0.25) (layer B.Cu) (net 24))
 (via (at 124.1125 99.2375) (size 0.8) (drill 0.4) (layers F.Cu B.Cu) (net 24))
 (segment (start 117.90625 99.25) (end 124.1 99.25) (width 0.25) (layer B.Cu) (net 24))
 (segment (start 126.2 94.9226) (end 126.2 98.7) (width 0.25) (layer F.Cu) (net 24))
 (segment (start 126.2 98.7) (end 125.6625 99.2375) (width 0.25) (layer F.Cu) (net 24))
 (segment (start 126.49375 94.62885) (end 126.2 94.9226) (width 0.25) (layer F.Cu) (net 24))
 (segment (start 125.6625 99.2375) (end 124.1125 99.2375) (width 0.25) (layer F.Cu) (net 24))
 (segment (start 126.49375 90.50625) (end 126.49375 94.62885) (width 0.25) (layer F.Cu) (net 24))
 (segment (start 127.9 89.1) (end 126.49375 90.50625) (width 0.25) (layer F.Cu) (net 24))
 (segment (start 148.10625 89.1) (end 127.9 89.1) (width 0.25) (layer F.Cu) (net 24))
 (segment (start 148.8775 89.87125) (end 148.10625 89.1) (width 0.25) (layer F.Cu) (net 24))
 (segment (start 148.8775 93.5225) (end 148.8775 89.87125) (width 0.25) (layer F.Cu) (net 24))
 (via (at 122.525 98.44375) (size 0.8) (drill 0.4) (layers F.Cu B.Cu) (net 25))
 (segment (start 122.51875 98.45) (end 122.525 98.44375) (width 0.25) (layer B.Cu) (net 25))
 (segment (start 117.90625 98.45) (end 122.51875 98.45) (width 0.25) (layer B.Cu) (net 25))
 (segment (start 125.15625 98.44375) (end 122.525 98.44375) (width 0.25) (layer F.Cu) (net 25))
 (segment (start 125.74999 97.85001) (end 125.15625 98.44375) (width 0.25) (layer F.Cu) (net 25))
 (segment (start 125.74999 94.7362) (end 125.74999 97.85001) (width 0.25) (layer F.Cu) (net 25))
 (segment (start 126.043741 94.442449) (end 125.74999 94.7362) (width 0.25) (layer F.Cu) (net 25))
 (segment (start 167.9275 89.6275) (end 166.9 88.6) (width 0.25) (layer F.Cu) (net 25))
 (segment (start 126.043741 90.319849) (end 126.043741 94.442449) (width 0.25) (layer F.Cu) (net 25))
 (segment (start 127.76359 88.6) (end 126.043741 90.319849) (width 0.25) (layer F.Cu) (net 25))
 (segment (start 166.9 88.6) (end 127.76359 88.6) (width 0.25) (layer F.Cu) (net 25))
 (segment (start 167.9275 93.5225) (end 167.9275 89.6275) (width 0.25) (layer F.Cu) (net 25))
 (via (at 124.1125 97.65) (size 0.8) (drill 0.4) (layers F.Cu B.Cu) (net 26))
 (segment (start 117.90625 97.65) (end 124.1125 97.65) (width 0.25) (layer B.Cu) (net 26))
 (segment (start 186.9775 93.5225) (end 186.9775 89.5775) (width 0.25) (layer F.Cu) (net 26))
 (segment (start 185.54999 88.14999) (end 127.577189 88.149991) (width 0.25) (layer F.Cu) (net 26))
 (segment (start 186.9775 89.5775) (end 185.54999 88.14999) (width 0.25) (layer F.Cu) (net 26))
 (segment (start 125.593731 94.256049) (end 125.29998 94.5498) (width 0.25) (layer F.Cu) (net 26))
 (segment (start 125.593731 90.133449) (end 125.593731 94.256049) (width 0.25) (layer F.Cu) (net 26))
 (segment (start 127.577189 88.149991) (end 125.593731 90.133449) (width 0.25) (layer F.Cu) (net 26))
 (segment (start 125.29998 94.5498) (end 125.29998 97.20002) (width 0.25) (layer F.Cu) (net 26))
 (segment (start 124.85 97.65) (end 124.1125 97.65) (width 0.25) (layer F.Cu) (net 26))
 (segment (start 125.29998 97.20002) (end 124.85 97.65) (width 0.25) (layer F.Cu) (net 26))
 (via (at 122.525 96.85625) (size 0.8) (drill 0.4) (layers F.Cu B.Cu) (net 27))
 (segment (start 122.51875 96.85) (end 122.525 96.85625) (width 0.25) (layer B.Cu) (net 27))
 (segment (start 117.90625 96.85) (end 122.51875 96.85) (width 0.25) (layer B.Cu) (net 27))
 (segment (start 122.593749 96.924999) (end 122.525 96.85625) (width 0.25) (layer F.Cu) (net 27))
 (segment (start 125.143721 89.947049) (end 125.143721 94.069649) (width 0.25) (layer F.Cu) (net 27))
 (segment (start 124.84997 94.3634) (end 124.84997 96.45003) (width 0.25) (layer F.Cu) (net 27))
 (segment (start 127.390788 87.699982) (end 125.143721 89.947049) (width 0.25) (layer F.Cu) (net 27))
 (segment (start 124.84997 96.45003) (end 124.375001 96.924999) (width 0.25) (layer F.Cu) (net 27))
 (segment (start 205.19998 87.699982) (end 127.390788 87.699982) (width 0.25) (layer F.Cu) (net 27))
 (segment (start 125.143721 94.069649) (end 124.84997 94.3634) (width 0.25) (layer F.Cu) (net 27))
 (segment (start 206.0275 88.5275) (end 205.19998 87.699982) (width 0.25) (layer F.Cu) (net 27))
 (segment (start 124.375001 96.924999) (end 122.593749 96.924999) (width 0.25) (layer F.Cu) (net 27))
 (segment (start 206.0275 93.5225) (end 206.0275 88.5275) (width 0.25) (layer F.Cu) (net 27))
 (via (at 124.1125 96.0625) (size 0.8) (drill 0.4) (layers F.Cu B.Cu) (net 2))
 (segment (start 124.1 96.05) (end 124.1125 96.0625) (width 0.25) (layer B.Cu) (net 2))
 (segment (start 117.90625 96.05) (end 124.1 96.05) (width 0.25) (layer B.Cu) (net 2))
 (segment (start 225.0775 93.5225) (end 225.0775 87.5775) (width 0.25) (layer F.Cu) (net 2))
 (segment (start 127.204387 87.249973) (end 124.693711 89.760649) (width 0.25) (layer F.Cu) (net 2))
 (segment (start 224.749972 87.249972) (end 127.204387 87.249973) (width 0.25) (layer F.Cu) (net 2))
 (segment (start 225.0775 87.5775) (end 224.749972 87.249972) (width 0.25) (layer F.Cu) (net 2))
 (segment (start 124.1125 94.46446) (end 124.1125 96.0625) (width 0.25) (layer F.Cu) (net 2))
 (segment (start 124.693711 93.883249) (end 124.1125 94.46446) (width 0.25) (layer F.Cu) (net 2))
 (segment (start 124.693711 89.760649) (end 124.693711 93.883249) (width 0.25) (layer F.Cu) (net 2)))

